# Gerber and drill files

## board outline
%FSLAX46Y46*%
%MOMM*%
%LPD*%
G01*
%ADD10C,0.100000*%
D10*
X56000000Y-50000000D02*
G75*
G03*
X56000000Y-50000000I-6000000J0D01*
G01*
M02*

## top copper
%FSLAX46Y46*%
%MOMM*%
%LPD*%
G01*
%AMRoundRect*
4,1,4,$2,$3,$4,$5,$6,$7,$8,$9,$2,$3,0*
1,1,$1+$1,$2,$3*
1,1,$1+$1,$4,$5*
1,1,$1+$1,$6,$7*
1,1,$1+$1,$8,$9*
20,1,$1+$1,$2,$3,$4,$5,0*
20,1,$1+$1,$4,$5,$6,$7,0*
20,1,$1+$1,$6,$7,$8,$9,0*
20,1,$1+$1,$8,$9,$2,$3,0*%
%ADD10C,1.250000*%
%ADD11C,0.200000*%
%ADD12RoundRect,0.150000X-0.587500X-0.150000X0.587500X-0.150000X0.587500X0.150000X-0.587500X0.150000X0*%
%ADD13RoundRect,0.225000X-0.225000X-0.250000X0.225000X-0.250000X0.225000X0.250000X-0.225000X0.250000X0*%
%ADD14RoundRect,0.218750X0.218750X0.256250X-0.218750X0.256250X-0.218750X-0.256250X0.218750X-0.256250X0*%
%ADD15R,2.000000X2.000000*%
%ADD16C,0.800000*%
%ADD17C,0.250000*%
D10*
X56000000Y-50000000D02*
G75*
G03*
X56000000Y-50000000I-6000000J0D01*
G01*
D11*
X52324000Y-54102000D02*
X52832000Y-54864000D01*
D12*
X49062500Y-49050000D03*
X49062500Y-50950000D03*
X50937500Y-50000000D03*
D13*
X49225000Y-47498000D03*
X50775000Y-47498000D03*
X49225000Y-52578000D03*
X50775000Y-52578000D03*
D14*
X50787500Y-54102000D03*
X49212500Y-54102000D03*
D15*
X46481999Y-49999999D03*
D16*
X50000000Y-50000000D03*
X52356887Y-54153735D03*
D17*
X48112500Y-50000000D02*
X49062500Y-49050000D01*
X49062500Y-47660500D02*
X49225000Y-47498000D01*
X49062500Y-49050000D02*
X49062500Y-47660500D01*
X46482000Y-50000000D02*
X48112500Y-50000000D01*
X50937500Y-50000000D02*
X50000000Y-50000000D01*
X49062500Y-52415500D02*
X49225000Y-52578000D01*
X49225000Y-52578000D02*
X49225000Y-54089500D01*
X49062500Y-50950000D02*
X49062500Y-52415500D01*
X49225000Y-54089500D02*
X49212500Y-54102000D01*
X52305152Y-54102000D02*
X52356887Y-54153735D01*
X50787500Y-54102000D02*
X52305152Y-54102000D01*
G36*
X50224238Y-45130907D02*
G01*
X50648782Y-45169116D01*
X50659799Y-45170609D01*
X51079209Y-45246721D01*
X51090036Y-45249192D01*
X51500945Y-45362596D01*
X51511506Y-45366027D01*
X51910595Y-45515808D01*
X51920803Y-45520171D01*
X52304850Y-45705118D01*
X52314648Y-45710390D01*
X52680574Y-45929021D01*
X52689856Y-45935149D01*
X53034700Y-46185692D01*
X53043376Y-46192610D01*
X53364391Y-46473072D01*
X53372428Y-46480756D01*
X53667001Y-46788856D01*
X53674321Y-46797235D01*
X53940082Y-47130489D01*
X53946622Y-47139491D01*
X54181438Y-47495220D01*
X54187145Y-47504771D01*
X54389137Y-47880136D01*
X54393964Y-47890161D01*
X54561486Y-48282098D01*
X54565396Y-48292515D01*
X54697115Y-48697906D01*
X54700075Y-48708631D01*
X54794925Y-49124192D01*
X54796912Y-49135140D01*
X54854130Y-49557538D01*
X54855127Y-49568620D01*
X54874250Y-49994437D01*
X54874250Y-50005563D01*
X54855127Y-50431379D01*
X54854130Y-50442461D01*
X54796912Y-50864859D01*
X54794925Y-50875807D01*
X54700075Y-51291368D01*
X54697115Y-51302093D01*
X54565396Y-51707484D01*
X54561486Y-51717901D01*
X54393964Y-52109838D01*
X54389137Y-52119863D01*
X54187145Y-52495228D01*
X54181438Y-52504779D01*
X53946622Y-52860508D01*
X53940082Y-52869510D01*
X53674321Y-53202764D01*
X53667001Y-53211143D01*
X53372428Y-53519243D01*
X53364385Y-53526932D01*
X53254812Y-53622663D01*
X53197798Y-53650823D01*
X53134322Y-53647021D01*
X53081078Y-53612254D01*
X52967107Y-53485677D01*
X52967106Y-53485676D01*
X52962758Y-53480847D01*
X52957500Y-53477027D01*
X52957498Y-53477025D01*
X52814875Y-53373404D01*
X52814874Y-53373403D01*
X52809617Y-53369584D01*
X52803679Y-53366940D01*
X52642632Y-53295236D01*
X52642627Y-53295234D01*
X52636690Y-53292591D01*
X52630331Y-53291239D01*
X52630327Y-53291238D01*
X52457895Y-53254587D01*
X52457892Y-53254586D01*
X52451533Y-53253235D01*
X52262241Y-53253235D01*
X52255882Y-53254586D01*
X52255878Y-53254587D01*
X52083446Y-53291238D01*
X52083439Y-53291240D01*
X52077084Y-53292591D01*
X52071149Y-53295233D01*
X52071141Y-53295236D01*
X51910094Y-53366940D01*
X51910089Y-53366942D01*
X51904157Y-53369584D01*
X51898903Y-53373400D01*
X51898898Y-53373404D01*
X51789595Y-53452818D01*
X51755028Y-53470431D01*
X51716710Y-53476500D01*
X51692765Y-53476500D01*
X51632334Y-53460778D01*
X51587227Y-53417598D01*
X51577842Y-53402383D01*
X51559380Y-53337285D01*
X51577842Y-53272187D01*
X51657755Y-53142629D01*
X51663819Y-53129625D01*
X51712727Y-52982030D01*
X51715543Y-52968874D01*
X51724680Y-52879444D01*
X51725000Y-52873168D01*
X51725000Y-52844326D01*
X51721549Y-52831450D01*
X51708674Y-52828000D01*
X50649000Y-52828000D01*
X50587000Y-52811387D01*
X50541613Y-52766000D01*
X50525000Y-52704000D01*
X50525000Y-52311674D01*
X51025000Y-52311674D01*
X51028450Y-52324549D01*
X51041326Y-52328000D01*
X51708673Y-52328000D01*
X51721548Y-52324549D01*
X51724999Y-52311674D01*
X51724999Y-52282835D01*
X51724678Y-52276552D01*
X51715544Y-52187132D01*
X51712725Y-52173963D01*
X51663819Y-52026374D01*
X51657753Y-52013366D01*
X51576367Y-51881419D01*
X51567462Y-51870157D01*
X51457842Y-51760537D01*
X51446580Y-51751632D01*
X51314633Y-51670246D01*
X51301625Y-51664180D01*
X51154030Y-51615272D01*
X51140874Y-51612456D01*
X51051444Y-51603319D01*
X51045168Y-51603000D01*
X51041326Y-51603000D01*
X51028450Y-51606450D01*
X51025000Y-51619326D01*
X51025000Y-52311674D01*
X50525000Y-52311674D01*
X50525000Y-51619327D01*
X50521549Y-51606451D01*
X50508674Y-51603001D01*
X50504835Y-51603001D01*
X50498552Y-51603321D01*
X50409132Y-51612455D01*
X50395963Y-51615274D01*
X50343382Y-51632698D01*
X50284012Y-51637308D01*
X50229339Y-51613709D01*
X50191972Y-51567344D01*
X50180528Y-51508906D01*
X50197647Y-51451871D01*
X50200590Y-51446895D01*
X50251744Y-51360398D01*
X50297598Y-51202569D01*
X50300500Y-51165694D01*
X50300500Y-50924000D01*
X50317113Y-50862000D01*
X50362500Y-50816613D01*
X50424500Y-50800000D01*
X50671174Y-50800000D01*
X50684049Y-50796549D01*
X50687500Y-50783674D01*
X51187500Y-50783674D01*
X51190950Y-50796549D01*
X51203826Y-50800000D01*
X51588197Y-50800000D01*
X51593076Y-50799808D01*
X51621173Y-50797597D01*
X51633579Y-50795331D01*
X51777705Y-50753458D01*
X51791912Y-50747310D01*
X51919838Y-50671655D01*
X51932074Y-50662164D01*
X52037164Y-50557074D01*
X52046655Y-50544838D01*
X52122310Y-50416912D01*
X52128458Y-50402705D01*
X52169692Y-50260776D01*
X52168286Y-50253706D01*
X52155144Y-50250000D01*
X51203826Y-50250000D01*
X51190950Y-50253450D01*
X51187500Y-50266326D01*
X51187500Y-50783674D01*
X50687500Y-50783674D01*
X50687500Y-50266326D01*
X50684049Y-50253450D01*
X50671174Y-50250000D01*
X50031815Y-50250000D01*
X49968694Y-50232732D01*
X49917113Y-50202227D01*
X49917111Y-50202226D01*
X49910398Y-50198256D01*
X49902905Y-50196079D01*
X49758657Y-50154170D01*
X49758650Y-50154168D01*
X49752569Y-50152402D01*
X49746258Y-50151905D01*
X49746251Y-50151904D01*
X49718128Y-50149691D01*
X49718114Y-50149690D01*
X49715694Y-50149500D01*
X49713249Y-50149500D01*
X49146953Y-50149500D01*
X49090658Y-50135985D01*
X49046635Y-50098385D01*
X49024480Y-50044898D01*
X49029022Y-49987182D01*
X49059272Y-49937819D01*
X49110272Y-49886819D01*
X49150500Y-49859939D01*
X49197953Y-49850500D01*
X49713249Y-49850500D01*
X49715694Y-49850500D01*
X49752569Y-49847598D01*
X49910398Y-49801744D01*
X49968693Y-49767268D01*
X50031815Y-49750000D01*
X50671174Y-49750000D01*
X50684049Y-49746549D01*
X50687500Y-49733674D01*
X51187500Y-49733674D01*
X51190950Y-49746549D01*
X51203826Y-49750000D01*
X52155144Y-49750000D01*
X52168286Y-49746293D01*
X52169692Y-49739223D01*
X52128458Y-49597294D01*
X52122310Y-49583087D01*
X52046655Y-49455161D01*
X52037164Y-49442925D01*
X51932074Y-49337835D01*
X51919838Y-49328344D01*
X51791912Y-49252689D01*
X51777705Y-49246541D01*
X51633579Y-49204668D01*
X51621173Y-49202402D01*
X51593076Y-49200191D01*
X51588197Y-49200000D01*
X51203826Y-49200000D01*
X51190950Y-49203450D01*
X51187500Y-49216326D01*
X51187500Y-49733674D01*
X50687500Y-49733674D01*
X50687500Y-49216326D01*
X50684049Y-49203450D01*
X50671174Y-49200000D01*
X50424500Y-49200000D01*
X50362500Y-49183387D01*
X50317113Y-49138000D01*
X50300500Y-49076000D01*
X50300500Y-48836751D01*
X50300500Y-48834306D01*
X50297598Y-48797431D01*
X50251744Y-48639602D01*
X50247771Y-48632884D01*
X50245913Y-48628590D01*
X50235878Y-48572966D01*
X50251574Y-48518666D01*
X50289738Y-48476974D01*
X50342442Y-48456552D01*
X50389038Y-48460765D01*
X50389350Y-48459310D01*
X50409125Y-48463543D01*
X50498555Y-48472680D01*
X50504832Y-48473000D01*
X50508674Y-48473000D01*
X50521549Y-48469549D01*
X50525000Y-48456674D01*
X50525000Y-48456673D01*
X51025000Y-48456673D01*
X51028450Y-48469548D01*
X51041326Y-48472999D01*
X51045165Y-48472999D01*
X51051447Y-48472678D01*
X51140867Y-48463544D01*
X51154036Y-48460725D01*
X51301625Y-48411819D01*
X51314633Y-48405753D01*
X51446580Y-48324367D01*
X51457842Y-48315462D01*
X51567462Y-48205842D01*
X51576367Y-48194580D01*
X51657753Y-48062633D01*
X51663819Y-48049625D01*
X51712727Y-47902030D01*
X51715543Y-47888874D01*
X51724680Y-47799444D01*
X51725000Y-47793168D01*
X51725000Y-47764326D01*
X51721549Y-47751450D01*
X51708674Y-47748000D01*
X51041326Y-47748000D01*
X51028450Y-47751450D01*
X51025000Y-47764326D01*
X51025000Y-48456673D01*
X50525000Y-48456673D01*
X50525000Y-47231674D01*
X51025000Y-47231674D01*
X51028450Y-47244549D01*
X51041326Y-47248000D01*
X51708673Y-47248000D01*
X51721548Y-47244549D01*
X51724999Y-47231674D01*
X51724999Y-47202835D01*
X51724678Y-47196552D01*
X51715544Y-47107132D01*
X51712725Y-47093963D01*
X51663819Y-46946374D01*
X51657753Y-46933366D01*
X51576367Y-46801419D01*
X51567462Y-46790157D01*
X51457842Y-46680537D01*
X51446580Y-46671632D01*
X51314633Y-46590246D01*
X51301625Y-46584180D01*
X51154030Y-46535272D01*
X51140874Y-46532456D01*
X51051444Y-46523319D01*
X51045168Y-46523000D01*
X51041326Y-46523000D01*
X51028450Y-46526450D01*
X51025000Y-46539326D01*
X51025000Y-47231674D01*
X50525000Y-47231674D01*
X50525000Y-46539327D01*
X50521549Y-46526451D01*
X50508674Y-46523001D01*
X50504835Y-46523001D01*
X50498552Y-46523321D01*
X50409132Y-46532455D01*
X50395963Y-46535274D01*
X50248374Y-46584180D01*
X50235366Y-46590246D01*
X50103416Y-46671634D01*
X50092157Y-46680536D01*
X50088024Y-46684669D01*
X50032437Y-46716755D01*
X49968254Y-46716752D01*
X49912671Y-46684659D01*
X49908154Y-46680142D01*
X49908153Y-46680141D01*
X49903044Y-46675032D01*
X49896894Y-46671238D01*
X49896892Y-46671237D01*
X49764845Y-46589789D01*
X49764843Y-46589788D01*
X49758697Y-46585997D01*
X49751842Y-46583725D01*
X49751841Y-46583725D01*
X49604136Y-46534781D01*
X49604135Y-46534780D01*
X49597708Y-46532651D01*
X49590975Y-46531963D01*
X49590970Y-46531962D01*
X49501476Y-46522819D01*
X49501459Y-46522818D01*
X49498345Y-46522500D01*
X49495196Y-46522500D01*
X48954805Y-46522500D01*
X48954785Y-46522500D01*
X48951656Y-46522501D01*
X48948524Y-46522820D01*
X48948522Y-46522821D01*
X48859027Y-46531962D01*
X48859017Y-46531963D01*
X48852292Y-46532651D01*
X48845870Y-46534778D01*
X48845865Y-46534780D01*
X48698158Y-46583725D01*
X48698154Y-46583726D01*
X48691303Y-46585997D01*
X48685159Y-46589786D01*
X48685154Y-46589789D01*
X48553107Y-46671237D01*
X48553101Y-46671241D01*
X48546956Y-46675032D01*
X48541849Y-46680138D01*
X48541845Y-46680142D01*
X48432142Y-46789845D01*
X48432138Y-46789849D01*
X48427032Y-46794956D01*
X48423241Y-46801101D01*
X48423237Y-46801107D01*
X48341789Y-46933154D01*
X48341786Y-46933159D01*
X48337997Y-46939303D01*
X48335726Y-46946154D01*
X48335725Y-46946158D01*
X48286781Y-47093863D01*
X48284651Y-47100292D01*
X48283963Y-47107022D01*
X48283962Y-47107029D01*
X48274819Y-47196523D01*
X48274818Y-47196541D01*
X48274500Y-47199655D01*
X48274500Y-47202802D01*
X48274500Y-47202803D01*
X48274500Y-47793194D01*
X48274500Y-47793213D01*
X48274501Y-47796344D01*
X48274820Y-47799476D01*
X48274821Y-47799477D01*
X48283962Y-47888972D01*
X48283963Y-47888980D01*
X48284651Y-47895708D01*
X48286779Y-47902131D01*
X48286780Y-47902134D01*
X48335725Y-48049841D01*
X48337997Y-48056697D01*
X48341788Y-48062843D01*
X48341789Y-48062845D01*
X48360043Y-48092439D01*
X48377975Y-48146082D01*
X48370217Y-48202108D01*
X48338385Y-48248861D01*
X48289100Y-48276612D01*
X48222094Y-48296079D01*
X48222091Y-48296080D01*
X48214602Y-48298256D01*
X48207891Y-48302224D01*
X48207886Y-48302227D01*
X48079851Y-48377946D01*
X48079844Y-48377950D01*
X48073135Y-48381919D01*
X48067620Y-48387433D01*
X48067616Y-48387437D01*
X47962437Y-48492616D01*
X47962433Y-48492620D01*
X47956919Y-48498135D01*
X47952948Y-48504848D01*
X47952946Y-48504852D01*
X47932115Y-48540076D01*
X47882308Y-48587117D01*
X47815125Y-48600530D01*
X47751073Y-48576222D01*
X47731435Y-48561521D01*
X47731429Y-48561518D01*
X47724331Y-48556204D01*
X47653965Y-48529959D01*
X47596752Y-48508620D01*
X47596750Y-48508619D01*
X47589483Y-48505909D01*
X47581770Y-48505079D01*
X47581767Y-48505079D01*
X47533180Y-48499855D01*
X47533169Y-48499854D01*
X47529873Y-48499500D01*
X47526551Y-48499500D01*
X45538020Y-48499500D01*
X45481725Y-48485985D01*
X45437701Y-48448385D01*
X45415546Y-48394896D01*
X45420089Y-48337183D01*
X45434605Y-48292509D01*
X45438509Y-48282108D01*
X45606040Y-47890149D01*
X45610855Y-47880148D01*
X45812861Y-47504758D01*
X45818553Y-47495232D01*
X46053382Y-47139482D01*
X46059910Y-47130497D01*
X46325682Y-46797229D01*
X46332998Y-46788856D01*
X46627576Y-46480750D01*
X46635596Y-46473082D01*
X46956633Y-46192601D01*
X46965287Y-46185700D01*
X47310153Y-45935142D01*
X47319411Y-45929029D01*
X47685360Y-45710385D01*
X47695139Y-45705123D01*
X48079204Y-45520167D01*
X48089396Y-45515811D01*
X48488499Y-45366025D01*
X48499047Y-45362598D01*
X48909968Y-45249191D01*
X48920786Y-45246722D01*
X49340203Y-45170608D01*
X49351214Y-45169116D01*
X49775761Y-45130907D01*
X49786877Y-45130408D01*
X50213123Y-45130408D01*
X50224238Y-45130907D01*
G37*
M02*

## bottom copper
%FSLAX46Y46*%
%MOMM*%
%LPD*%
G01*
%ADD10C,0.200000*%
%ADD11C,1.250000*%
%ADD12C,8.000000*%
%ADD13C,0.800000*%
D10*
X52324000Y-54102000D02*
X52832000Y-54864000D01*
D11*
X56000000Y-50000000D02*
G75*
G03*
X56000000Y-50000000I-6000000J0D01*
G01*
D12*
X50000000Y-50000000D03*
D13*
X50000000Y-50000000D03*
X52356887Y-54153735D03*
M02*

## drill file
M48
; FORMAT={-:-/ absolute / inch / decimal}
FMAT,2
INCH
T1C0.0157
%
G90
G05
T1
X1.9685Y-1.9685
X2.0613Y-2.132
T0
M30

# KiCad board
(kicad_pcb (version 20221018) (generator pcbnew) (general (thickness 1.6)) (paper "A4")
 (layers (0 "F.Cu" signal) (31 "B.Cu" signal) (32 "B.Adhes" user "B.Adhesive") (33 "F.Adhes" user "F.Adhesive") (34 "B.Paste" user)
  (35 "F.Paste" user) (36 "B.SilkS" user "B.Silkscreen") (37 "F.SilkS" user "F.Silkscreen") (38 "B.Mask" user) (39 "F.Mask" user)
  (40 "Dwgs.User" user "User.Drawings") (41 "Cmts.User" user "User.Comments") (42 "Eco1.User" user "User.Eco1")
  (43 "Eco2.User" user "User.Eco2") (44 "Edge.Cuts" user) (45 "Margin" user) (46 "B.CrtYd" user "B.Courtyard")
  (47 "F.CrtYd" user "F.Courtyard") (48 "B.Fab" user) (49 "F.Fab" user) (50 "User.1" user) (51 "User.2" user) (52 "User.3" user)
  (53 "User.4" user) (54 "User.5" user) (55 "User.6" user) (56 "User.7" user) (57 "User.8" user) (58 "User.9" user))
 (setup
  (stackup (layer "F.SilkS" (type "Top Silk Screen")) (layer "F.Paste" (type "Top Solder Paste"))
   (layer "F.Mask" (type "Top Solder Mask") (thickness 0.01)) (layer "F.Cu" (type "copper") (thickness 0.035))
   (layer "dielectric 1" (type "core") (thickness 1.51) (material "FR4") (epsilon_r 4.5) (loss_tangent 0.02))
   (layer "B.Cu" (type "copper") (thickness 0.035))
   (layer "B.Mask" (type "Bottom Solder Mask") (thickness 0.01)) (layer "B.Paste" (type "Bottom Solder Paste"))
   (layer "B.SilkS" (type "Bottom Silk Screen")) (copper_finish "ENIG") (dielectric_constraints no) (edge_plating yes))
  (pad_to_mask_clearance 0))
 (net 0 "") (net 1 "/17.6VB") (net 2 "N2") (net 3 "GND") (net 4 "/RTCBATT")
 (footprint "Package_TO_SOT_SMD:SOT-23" (layer "F.Cu") (at 50 50)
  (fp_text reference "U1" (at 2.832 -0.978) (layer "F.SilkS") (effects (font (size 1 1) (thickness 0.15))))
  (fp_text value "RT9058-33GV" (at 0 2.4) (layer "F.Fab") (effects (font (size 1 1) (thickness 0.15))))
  (pad "1" smd roundrect (at -0.9375 -0.95) (size 1.475 0.6) (layers "F.Cu" "F.Paste" "F.Mask") (roundrect_rratio 0.25) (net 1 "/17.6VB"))
  (pad "2" smd roundrect (at -0.9375 0.95) (size 1.475 0.6) (layers "F.Cu" "F.Paste" "F.Mask") (roundrect_rratio 0.25) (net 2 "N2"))
  (pad "3" smd roundrect (at 0.9375 0) (size 1.475 0.6) (layers "F.Cu" "F.Paste" "F.Mask") (roundrect_rratio 0.25) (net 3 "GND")))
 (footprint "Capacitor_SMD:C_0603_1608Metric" (layer "F.Cu") (at 50 47.498)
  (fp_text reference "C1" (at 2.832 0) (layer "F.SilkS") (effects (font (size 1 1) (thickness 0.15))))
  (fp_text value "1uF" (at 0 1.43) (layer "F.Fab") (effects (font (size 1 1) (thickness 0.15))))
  (pad "1" smd roundrect (at -0.775 0) (size 0.9 0.95) (layers "F.Cu" "F.Paste" "F.Mask") (roundrect_rratio 0.25) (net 1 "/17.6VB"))
  (pad "2" smd roundrect (at 0.775 0) (size 0.9 0.95) (layers "F.Cu" "F.Paste" "F.Mask") (roundrect_rratio 0.25) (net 3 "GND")))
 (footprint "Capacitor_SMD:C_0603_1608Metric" (layer "F.Cu") (at 50 52.578)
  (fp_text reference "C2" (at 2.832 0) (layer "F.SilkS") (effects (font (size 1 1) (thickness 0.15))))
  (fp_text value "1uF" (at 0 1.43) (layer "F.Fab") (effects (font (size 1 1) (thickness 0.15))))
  (pad "1" smd roundrect (at -0.775 0) (size 0.9 0.95) (layers "F.Cu" "F.Paste" "F.Mask") (roundrect_rratio 0.25) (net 2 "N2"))
  (pad "2" smd roundrect (at 0.775 0) (size 0.9 0.95) (layers "F.Cu" "F.Paste" "F.Mask") (roundrect_rratio 0.25) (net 3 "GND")))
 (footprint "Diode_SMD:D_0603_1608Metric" (layer "F.Cu") (at 50 54.102 180)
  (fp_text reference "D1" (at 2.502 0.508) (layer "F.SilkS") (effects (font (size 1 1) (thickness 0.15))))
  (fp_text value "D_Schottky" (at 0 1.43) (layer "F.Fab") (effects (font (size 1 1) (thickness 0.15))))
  (pad "1" smd roundrect (at -0.7875 0 180) (size 0.875 0.95) (layers "F.Cu" "F.Paste" "F.Mask") (roundrect_rratio 0.25) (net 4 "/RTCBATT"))
  (pad "2" smd roundrect (at 0.7875 0 180) (size 0.875 0.95) (layers "F.Cu" "F.Paste" "F.Mask") (roundrect_rratio 0.25) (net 2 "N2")))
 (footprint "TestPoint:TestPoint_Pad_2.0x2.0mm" (layer "F.Cu") (at 46.482 50)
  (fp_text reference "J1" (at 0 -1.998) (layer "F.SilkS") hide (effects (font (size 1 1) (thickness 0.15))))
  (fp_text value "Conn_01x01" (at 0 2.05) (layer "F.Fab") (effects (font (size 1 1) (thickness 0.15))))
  (pad "1" smd rect (at 0 0) (size 2 2) (layers "F.Cu" "F.Mask") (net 1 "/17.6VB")))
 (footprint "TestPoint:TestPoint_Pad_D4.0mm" (layer "B.Cu") (at 50 50 180)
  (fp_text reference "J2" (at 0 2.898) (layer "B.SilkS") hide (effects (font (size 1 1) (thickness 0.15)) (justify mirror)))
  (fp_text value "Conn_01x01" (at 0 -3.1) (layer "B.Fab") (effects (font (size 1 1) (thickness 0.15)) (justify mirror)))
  (pad "1" smd circle (at 0 0 180) (size 8 8) (layers "B.Cu" "B.Mask") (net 3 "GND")))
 (gr_circle (center 50 50) (end 56 50) (stroke (width 1.25) (type solid)) (fill none) (layer "F.Cu"))
 (gr_line (start 52.324 54.102) (end 52.832 54.864) (stroke (width 0.2) (type default)) (layer "F.Cu"))
 (gr_line (start 52.324 54.102) (end 52.832 54.864) (stroke (width 0.2) (type default)) (layer "B.Cu"))
 (gr_circle (center 50 50) (end 56 50) (stroke (width 1.25) (type solid)) (fill none) (layer "B.Cu"))
 (gr_circle (center 50 50) (end 56 50) (stroke (width 0.1) (type default)) (fill none) (layer "Edge.Cuts"))
 (segment (start 48.1125 50) (end 49.0625 49.05) (width 0.25) (layer "F.Cu") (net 1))
 (segment (start 49.0625 47.6605) (end 49.225 47.498) (width 0.25) (layer "F.Cu") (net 1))
 (segment (start 49.0625 49.05) (end 49.0625 47.6605) (width 0.25) (layer "F.Cu") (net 1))
 (segment (start 46.482 50) (end 48.1125 50) (width 0.25) (layer "F.Cu") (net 1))
 (segment (start 50.9375 50) (end 50 50) (width 0.25) (layer "F.Cu") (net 3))
 (via (at 50 50) (size 0.8) (drill 0.4) (layers "F.Cu" "B.Cu") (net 3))
 (segment (start 49.0625 52.4155) (end 49.225 52.578) (width 0.25) (layer "F.Cu") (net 2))
 (segment (start 49.225 52.578) (end 49.225 54.0895) (width 0.25) (layer "F.Cu") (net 2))
 (segment (start 49.0625 50.95) (end 49.0625 52.4155) (width 0.25) (layer "F.Cu") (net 2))
 (segment (start 49.225 54.0895) (end 49.2125 54.102) (width 0.25) (layer "F.Cu") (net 2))
 (segment (start 52.305152 54.102) (end 52.356887 54.153735) (width 0.25) (layer "F.Cu") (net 4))
 (segment (start 50.7875 54.102) (end 52.305152 54.102) (width 0.25) (layer "F.Cu") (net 4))
 (via (at 52.356887 54.153735) (size 0.8) (drill 0.4) (layers "F.Cu" "B.Cu") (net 4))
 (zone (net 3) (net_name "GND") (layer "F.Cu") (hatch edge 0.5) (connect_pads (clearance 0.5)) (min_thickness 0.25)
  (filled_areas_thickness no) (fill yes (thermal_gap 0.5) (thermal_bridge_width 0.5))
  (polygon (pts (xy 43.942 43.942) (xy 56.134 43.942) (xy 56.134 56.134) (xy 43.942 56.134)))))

